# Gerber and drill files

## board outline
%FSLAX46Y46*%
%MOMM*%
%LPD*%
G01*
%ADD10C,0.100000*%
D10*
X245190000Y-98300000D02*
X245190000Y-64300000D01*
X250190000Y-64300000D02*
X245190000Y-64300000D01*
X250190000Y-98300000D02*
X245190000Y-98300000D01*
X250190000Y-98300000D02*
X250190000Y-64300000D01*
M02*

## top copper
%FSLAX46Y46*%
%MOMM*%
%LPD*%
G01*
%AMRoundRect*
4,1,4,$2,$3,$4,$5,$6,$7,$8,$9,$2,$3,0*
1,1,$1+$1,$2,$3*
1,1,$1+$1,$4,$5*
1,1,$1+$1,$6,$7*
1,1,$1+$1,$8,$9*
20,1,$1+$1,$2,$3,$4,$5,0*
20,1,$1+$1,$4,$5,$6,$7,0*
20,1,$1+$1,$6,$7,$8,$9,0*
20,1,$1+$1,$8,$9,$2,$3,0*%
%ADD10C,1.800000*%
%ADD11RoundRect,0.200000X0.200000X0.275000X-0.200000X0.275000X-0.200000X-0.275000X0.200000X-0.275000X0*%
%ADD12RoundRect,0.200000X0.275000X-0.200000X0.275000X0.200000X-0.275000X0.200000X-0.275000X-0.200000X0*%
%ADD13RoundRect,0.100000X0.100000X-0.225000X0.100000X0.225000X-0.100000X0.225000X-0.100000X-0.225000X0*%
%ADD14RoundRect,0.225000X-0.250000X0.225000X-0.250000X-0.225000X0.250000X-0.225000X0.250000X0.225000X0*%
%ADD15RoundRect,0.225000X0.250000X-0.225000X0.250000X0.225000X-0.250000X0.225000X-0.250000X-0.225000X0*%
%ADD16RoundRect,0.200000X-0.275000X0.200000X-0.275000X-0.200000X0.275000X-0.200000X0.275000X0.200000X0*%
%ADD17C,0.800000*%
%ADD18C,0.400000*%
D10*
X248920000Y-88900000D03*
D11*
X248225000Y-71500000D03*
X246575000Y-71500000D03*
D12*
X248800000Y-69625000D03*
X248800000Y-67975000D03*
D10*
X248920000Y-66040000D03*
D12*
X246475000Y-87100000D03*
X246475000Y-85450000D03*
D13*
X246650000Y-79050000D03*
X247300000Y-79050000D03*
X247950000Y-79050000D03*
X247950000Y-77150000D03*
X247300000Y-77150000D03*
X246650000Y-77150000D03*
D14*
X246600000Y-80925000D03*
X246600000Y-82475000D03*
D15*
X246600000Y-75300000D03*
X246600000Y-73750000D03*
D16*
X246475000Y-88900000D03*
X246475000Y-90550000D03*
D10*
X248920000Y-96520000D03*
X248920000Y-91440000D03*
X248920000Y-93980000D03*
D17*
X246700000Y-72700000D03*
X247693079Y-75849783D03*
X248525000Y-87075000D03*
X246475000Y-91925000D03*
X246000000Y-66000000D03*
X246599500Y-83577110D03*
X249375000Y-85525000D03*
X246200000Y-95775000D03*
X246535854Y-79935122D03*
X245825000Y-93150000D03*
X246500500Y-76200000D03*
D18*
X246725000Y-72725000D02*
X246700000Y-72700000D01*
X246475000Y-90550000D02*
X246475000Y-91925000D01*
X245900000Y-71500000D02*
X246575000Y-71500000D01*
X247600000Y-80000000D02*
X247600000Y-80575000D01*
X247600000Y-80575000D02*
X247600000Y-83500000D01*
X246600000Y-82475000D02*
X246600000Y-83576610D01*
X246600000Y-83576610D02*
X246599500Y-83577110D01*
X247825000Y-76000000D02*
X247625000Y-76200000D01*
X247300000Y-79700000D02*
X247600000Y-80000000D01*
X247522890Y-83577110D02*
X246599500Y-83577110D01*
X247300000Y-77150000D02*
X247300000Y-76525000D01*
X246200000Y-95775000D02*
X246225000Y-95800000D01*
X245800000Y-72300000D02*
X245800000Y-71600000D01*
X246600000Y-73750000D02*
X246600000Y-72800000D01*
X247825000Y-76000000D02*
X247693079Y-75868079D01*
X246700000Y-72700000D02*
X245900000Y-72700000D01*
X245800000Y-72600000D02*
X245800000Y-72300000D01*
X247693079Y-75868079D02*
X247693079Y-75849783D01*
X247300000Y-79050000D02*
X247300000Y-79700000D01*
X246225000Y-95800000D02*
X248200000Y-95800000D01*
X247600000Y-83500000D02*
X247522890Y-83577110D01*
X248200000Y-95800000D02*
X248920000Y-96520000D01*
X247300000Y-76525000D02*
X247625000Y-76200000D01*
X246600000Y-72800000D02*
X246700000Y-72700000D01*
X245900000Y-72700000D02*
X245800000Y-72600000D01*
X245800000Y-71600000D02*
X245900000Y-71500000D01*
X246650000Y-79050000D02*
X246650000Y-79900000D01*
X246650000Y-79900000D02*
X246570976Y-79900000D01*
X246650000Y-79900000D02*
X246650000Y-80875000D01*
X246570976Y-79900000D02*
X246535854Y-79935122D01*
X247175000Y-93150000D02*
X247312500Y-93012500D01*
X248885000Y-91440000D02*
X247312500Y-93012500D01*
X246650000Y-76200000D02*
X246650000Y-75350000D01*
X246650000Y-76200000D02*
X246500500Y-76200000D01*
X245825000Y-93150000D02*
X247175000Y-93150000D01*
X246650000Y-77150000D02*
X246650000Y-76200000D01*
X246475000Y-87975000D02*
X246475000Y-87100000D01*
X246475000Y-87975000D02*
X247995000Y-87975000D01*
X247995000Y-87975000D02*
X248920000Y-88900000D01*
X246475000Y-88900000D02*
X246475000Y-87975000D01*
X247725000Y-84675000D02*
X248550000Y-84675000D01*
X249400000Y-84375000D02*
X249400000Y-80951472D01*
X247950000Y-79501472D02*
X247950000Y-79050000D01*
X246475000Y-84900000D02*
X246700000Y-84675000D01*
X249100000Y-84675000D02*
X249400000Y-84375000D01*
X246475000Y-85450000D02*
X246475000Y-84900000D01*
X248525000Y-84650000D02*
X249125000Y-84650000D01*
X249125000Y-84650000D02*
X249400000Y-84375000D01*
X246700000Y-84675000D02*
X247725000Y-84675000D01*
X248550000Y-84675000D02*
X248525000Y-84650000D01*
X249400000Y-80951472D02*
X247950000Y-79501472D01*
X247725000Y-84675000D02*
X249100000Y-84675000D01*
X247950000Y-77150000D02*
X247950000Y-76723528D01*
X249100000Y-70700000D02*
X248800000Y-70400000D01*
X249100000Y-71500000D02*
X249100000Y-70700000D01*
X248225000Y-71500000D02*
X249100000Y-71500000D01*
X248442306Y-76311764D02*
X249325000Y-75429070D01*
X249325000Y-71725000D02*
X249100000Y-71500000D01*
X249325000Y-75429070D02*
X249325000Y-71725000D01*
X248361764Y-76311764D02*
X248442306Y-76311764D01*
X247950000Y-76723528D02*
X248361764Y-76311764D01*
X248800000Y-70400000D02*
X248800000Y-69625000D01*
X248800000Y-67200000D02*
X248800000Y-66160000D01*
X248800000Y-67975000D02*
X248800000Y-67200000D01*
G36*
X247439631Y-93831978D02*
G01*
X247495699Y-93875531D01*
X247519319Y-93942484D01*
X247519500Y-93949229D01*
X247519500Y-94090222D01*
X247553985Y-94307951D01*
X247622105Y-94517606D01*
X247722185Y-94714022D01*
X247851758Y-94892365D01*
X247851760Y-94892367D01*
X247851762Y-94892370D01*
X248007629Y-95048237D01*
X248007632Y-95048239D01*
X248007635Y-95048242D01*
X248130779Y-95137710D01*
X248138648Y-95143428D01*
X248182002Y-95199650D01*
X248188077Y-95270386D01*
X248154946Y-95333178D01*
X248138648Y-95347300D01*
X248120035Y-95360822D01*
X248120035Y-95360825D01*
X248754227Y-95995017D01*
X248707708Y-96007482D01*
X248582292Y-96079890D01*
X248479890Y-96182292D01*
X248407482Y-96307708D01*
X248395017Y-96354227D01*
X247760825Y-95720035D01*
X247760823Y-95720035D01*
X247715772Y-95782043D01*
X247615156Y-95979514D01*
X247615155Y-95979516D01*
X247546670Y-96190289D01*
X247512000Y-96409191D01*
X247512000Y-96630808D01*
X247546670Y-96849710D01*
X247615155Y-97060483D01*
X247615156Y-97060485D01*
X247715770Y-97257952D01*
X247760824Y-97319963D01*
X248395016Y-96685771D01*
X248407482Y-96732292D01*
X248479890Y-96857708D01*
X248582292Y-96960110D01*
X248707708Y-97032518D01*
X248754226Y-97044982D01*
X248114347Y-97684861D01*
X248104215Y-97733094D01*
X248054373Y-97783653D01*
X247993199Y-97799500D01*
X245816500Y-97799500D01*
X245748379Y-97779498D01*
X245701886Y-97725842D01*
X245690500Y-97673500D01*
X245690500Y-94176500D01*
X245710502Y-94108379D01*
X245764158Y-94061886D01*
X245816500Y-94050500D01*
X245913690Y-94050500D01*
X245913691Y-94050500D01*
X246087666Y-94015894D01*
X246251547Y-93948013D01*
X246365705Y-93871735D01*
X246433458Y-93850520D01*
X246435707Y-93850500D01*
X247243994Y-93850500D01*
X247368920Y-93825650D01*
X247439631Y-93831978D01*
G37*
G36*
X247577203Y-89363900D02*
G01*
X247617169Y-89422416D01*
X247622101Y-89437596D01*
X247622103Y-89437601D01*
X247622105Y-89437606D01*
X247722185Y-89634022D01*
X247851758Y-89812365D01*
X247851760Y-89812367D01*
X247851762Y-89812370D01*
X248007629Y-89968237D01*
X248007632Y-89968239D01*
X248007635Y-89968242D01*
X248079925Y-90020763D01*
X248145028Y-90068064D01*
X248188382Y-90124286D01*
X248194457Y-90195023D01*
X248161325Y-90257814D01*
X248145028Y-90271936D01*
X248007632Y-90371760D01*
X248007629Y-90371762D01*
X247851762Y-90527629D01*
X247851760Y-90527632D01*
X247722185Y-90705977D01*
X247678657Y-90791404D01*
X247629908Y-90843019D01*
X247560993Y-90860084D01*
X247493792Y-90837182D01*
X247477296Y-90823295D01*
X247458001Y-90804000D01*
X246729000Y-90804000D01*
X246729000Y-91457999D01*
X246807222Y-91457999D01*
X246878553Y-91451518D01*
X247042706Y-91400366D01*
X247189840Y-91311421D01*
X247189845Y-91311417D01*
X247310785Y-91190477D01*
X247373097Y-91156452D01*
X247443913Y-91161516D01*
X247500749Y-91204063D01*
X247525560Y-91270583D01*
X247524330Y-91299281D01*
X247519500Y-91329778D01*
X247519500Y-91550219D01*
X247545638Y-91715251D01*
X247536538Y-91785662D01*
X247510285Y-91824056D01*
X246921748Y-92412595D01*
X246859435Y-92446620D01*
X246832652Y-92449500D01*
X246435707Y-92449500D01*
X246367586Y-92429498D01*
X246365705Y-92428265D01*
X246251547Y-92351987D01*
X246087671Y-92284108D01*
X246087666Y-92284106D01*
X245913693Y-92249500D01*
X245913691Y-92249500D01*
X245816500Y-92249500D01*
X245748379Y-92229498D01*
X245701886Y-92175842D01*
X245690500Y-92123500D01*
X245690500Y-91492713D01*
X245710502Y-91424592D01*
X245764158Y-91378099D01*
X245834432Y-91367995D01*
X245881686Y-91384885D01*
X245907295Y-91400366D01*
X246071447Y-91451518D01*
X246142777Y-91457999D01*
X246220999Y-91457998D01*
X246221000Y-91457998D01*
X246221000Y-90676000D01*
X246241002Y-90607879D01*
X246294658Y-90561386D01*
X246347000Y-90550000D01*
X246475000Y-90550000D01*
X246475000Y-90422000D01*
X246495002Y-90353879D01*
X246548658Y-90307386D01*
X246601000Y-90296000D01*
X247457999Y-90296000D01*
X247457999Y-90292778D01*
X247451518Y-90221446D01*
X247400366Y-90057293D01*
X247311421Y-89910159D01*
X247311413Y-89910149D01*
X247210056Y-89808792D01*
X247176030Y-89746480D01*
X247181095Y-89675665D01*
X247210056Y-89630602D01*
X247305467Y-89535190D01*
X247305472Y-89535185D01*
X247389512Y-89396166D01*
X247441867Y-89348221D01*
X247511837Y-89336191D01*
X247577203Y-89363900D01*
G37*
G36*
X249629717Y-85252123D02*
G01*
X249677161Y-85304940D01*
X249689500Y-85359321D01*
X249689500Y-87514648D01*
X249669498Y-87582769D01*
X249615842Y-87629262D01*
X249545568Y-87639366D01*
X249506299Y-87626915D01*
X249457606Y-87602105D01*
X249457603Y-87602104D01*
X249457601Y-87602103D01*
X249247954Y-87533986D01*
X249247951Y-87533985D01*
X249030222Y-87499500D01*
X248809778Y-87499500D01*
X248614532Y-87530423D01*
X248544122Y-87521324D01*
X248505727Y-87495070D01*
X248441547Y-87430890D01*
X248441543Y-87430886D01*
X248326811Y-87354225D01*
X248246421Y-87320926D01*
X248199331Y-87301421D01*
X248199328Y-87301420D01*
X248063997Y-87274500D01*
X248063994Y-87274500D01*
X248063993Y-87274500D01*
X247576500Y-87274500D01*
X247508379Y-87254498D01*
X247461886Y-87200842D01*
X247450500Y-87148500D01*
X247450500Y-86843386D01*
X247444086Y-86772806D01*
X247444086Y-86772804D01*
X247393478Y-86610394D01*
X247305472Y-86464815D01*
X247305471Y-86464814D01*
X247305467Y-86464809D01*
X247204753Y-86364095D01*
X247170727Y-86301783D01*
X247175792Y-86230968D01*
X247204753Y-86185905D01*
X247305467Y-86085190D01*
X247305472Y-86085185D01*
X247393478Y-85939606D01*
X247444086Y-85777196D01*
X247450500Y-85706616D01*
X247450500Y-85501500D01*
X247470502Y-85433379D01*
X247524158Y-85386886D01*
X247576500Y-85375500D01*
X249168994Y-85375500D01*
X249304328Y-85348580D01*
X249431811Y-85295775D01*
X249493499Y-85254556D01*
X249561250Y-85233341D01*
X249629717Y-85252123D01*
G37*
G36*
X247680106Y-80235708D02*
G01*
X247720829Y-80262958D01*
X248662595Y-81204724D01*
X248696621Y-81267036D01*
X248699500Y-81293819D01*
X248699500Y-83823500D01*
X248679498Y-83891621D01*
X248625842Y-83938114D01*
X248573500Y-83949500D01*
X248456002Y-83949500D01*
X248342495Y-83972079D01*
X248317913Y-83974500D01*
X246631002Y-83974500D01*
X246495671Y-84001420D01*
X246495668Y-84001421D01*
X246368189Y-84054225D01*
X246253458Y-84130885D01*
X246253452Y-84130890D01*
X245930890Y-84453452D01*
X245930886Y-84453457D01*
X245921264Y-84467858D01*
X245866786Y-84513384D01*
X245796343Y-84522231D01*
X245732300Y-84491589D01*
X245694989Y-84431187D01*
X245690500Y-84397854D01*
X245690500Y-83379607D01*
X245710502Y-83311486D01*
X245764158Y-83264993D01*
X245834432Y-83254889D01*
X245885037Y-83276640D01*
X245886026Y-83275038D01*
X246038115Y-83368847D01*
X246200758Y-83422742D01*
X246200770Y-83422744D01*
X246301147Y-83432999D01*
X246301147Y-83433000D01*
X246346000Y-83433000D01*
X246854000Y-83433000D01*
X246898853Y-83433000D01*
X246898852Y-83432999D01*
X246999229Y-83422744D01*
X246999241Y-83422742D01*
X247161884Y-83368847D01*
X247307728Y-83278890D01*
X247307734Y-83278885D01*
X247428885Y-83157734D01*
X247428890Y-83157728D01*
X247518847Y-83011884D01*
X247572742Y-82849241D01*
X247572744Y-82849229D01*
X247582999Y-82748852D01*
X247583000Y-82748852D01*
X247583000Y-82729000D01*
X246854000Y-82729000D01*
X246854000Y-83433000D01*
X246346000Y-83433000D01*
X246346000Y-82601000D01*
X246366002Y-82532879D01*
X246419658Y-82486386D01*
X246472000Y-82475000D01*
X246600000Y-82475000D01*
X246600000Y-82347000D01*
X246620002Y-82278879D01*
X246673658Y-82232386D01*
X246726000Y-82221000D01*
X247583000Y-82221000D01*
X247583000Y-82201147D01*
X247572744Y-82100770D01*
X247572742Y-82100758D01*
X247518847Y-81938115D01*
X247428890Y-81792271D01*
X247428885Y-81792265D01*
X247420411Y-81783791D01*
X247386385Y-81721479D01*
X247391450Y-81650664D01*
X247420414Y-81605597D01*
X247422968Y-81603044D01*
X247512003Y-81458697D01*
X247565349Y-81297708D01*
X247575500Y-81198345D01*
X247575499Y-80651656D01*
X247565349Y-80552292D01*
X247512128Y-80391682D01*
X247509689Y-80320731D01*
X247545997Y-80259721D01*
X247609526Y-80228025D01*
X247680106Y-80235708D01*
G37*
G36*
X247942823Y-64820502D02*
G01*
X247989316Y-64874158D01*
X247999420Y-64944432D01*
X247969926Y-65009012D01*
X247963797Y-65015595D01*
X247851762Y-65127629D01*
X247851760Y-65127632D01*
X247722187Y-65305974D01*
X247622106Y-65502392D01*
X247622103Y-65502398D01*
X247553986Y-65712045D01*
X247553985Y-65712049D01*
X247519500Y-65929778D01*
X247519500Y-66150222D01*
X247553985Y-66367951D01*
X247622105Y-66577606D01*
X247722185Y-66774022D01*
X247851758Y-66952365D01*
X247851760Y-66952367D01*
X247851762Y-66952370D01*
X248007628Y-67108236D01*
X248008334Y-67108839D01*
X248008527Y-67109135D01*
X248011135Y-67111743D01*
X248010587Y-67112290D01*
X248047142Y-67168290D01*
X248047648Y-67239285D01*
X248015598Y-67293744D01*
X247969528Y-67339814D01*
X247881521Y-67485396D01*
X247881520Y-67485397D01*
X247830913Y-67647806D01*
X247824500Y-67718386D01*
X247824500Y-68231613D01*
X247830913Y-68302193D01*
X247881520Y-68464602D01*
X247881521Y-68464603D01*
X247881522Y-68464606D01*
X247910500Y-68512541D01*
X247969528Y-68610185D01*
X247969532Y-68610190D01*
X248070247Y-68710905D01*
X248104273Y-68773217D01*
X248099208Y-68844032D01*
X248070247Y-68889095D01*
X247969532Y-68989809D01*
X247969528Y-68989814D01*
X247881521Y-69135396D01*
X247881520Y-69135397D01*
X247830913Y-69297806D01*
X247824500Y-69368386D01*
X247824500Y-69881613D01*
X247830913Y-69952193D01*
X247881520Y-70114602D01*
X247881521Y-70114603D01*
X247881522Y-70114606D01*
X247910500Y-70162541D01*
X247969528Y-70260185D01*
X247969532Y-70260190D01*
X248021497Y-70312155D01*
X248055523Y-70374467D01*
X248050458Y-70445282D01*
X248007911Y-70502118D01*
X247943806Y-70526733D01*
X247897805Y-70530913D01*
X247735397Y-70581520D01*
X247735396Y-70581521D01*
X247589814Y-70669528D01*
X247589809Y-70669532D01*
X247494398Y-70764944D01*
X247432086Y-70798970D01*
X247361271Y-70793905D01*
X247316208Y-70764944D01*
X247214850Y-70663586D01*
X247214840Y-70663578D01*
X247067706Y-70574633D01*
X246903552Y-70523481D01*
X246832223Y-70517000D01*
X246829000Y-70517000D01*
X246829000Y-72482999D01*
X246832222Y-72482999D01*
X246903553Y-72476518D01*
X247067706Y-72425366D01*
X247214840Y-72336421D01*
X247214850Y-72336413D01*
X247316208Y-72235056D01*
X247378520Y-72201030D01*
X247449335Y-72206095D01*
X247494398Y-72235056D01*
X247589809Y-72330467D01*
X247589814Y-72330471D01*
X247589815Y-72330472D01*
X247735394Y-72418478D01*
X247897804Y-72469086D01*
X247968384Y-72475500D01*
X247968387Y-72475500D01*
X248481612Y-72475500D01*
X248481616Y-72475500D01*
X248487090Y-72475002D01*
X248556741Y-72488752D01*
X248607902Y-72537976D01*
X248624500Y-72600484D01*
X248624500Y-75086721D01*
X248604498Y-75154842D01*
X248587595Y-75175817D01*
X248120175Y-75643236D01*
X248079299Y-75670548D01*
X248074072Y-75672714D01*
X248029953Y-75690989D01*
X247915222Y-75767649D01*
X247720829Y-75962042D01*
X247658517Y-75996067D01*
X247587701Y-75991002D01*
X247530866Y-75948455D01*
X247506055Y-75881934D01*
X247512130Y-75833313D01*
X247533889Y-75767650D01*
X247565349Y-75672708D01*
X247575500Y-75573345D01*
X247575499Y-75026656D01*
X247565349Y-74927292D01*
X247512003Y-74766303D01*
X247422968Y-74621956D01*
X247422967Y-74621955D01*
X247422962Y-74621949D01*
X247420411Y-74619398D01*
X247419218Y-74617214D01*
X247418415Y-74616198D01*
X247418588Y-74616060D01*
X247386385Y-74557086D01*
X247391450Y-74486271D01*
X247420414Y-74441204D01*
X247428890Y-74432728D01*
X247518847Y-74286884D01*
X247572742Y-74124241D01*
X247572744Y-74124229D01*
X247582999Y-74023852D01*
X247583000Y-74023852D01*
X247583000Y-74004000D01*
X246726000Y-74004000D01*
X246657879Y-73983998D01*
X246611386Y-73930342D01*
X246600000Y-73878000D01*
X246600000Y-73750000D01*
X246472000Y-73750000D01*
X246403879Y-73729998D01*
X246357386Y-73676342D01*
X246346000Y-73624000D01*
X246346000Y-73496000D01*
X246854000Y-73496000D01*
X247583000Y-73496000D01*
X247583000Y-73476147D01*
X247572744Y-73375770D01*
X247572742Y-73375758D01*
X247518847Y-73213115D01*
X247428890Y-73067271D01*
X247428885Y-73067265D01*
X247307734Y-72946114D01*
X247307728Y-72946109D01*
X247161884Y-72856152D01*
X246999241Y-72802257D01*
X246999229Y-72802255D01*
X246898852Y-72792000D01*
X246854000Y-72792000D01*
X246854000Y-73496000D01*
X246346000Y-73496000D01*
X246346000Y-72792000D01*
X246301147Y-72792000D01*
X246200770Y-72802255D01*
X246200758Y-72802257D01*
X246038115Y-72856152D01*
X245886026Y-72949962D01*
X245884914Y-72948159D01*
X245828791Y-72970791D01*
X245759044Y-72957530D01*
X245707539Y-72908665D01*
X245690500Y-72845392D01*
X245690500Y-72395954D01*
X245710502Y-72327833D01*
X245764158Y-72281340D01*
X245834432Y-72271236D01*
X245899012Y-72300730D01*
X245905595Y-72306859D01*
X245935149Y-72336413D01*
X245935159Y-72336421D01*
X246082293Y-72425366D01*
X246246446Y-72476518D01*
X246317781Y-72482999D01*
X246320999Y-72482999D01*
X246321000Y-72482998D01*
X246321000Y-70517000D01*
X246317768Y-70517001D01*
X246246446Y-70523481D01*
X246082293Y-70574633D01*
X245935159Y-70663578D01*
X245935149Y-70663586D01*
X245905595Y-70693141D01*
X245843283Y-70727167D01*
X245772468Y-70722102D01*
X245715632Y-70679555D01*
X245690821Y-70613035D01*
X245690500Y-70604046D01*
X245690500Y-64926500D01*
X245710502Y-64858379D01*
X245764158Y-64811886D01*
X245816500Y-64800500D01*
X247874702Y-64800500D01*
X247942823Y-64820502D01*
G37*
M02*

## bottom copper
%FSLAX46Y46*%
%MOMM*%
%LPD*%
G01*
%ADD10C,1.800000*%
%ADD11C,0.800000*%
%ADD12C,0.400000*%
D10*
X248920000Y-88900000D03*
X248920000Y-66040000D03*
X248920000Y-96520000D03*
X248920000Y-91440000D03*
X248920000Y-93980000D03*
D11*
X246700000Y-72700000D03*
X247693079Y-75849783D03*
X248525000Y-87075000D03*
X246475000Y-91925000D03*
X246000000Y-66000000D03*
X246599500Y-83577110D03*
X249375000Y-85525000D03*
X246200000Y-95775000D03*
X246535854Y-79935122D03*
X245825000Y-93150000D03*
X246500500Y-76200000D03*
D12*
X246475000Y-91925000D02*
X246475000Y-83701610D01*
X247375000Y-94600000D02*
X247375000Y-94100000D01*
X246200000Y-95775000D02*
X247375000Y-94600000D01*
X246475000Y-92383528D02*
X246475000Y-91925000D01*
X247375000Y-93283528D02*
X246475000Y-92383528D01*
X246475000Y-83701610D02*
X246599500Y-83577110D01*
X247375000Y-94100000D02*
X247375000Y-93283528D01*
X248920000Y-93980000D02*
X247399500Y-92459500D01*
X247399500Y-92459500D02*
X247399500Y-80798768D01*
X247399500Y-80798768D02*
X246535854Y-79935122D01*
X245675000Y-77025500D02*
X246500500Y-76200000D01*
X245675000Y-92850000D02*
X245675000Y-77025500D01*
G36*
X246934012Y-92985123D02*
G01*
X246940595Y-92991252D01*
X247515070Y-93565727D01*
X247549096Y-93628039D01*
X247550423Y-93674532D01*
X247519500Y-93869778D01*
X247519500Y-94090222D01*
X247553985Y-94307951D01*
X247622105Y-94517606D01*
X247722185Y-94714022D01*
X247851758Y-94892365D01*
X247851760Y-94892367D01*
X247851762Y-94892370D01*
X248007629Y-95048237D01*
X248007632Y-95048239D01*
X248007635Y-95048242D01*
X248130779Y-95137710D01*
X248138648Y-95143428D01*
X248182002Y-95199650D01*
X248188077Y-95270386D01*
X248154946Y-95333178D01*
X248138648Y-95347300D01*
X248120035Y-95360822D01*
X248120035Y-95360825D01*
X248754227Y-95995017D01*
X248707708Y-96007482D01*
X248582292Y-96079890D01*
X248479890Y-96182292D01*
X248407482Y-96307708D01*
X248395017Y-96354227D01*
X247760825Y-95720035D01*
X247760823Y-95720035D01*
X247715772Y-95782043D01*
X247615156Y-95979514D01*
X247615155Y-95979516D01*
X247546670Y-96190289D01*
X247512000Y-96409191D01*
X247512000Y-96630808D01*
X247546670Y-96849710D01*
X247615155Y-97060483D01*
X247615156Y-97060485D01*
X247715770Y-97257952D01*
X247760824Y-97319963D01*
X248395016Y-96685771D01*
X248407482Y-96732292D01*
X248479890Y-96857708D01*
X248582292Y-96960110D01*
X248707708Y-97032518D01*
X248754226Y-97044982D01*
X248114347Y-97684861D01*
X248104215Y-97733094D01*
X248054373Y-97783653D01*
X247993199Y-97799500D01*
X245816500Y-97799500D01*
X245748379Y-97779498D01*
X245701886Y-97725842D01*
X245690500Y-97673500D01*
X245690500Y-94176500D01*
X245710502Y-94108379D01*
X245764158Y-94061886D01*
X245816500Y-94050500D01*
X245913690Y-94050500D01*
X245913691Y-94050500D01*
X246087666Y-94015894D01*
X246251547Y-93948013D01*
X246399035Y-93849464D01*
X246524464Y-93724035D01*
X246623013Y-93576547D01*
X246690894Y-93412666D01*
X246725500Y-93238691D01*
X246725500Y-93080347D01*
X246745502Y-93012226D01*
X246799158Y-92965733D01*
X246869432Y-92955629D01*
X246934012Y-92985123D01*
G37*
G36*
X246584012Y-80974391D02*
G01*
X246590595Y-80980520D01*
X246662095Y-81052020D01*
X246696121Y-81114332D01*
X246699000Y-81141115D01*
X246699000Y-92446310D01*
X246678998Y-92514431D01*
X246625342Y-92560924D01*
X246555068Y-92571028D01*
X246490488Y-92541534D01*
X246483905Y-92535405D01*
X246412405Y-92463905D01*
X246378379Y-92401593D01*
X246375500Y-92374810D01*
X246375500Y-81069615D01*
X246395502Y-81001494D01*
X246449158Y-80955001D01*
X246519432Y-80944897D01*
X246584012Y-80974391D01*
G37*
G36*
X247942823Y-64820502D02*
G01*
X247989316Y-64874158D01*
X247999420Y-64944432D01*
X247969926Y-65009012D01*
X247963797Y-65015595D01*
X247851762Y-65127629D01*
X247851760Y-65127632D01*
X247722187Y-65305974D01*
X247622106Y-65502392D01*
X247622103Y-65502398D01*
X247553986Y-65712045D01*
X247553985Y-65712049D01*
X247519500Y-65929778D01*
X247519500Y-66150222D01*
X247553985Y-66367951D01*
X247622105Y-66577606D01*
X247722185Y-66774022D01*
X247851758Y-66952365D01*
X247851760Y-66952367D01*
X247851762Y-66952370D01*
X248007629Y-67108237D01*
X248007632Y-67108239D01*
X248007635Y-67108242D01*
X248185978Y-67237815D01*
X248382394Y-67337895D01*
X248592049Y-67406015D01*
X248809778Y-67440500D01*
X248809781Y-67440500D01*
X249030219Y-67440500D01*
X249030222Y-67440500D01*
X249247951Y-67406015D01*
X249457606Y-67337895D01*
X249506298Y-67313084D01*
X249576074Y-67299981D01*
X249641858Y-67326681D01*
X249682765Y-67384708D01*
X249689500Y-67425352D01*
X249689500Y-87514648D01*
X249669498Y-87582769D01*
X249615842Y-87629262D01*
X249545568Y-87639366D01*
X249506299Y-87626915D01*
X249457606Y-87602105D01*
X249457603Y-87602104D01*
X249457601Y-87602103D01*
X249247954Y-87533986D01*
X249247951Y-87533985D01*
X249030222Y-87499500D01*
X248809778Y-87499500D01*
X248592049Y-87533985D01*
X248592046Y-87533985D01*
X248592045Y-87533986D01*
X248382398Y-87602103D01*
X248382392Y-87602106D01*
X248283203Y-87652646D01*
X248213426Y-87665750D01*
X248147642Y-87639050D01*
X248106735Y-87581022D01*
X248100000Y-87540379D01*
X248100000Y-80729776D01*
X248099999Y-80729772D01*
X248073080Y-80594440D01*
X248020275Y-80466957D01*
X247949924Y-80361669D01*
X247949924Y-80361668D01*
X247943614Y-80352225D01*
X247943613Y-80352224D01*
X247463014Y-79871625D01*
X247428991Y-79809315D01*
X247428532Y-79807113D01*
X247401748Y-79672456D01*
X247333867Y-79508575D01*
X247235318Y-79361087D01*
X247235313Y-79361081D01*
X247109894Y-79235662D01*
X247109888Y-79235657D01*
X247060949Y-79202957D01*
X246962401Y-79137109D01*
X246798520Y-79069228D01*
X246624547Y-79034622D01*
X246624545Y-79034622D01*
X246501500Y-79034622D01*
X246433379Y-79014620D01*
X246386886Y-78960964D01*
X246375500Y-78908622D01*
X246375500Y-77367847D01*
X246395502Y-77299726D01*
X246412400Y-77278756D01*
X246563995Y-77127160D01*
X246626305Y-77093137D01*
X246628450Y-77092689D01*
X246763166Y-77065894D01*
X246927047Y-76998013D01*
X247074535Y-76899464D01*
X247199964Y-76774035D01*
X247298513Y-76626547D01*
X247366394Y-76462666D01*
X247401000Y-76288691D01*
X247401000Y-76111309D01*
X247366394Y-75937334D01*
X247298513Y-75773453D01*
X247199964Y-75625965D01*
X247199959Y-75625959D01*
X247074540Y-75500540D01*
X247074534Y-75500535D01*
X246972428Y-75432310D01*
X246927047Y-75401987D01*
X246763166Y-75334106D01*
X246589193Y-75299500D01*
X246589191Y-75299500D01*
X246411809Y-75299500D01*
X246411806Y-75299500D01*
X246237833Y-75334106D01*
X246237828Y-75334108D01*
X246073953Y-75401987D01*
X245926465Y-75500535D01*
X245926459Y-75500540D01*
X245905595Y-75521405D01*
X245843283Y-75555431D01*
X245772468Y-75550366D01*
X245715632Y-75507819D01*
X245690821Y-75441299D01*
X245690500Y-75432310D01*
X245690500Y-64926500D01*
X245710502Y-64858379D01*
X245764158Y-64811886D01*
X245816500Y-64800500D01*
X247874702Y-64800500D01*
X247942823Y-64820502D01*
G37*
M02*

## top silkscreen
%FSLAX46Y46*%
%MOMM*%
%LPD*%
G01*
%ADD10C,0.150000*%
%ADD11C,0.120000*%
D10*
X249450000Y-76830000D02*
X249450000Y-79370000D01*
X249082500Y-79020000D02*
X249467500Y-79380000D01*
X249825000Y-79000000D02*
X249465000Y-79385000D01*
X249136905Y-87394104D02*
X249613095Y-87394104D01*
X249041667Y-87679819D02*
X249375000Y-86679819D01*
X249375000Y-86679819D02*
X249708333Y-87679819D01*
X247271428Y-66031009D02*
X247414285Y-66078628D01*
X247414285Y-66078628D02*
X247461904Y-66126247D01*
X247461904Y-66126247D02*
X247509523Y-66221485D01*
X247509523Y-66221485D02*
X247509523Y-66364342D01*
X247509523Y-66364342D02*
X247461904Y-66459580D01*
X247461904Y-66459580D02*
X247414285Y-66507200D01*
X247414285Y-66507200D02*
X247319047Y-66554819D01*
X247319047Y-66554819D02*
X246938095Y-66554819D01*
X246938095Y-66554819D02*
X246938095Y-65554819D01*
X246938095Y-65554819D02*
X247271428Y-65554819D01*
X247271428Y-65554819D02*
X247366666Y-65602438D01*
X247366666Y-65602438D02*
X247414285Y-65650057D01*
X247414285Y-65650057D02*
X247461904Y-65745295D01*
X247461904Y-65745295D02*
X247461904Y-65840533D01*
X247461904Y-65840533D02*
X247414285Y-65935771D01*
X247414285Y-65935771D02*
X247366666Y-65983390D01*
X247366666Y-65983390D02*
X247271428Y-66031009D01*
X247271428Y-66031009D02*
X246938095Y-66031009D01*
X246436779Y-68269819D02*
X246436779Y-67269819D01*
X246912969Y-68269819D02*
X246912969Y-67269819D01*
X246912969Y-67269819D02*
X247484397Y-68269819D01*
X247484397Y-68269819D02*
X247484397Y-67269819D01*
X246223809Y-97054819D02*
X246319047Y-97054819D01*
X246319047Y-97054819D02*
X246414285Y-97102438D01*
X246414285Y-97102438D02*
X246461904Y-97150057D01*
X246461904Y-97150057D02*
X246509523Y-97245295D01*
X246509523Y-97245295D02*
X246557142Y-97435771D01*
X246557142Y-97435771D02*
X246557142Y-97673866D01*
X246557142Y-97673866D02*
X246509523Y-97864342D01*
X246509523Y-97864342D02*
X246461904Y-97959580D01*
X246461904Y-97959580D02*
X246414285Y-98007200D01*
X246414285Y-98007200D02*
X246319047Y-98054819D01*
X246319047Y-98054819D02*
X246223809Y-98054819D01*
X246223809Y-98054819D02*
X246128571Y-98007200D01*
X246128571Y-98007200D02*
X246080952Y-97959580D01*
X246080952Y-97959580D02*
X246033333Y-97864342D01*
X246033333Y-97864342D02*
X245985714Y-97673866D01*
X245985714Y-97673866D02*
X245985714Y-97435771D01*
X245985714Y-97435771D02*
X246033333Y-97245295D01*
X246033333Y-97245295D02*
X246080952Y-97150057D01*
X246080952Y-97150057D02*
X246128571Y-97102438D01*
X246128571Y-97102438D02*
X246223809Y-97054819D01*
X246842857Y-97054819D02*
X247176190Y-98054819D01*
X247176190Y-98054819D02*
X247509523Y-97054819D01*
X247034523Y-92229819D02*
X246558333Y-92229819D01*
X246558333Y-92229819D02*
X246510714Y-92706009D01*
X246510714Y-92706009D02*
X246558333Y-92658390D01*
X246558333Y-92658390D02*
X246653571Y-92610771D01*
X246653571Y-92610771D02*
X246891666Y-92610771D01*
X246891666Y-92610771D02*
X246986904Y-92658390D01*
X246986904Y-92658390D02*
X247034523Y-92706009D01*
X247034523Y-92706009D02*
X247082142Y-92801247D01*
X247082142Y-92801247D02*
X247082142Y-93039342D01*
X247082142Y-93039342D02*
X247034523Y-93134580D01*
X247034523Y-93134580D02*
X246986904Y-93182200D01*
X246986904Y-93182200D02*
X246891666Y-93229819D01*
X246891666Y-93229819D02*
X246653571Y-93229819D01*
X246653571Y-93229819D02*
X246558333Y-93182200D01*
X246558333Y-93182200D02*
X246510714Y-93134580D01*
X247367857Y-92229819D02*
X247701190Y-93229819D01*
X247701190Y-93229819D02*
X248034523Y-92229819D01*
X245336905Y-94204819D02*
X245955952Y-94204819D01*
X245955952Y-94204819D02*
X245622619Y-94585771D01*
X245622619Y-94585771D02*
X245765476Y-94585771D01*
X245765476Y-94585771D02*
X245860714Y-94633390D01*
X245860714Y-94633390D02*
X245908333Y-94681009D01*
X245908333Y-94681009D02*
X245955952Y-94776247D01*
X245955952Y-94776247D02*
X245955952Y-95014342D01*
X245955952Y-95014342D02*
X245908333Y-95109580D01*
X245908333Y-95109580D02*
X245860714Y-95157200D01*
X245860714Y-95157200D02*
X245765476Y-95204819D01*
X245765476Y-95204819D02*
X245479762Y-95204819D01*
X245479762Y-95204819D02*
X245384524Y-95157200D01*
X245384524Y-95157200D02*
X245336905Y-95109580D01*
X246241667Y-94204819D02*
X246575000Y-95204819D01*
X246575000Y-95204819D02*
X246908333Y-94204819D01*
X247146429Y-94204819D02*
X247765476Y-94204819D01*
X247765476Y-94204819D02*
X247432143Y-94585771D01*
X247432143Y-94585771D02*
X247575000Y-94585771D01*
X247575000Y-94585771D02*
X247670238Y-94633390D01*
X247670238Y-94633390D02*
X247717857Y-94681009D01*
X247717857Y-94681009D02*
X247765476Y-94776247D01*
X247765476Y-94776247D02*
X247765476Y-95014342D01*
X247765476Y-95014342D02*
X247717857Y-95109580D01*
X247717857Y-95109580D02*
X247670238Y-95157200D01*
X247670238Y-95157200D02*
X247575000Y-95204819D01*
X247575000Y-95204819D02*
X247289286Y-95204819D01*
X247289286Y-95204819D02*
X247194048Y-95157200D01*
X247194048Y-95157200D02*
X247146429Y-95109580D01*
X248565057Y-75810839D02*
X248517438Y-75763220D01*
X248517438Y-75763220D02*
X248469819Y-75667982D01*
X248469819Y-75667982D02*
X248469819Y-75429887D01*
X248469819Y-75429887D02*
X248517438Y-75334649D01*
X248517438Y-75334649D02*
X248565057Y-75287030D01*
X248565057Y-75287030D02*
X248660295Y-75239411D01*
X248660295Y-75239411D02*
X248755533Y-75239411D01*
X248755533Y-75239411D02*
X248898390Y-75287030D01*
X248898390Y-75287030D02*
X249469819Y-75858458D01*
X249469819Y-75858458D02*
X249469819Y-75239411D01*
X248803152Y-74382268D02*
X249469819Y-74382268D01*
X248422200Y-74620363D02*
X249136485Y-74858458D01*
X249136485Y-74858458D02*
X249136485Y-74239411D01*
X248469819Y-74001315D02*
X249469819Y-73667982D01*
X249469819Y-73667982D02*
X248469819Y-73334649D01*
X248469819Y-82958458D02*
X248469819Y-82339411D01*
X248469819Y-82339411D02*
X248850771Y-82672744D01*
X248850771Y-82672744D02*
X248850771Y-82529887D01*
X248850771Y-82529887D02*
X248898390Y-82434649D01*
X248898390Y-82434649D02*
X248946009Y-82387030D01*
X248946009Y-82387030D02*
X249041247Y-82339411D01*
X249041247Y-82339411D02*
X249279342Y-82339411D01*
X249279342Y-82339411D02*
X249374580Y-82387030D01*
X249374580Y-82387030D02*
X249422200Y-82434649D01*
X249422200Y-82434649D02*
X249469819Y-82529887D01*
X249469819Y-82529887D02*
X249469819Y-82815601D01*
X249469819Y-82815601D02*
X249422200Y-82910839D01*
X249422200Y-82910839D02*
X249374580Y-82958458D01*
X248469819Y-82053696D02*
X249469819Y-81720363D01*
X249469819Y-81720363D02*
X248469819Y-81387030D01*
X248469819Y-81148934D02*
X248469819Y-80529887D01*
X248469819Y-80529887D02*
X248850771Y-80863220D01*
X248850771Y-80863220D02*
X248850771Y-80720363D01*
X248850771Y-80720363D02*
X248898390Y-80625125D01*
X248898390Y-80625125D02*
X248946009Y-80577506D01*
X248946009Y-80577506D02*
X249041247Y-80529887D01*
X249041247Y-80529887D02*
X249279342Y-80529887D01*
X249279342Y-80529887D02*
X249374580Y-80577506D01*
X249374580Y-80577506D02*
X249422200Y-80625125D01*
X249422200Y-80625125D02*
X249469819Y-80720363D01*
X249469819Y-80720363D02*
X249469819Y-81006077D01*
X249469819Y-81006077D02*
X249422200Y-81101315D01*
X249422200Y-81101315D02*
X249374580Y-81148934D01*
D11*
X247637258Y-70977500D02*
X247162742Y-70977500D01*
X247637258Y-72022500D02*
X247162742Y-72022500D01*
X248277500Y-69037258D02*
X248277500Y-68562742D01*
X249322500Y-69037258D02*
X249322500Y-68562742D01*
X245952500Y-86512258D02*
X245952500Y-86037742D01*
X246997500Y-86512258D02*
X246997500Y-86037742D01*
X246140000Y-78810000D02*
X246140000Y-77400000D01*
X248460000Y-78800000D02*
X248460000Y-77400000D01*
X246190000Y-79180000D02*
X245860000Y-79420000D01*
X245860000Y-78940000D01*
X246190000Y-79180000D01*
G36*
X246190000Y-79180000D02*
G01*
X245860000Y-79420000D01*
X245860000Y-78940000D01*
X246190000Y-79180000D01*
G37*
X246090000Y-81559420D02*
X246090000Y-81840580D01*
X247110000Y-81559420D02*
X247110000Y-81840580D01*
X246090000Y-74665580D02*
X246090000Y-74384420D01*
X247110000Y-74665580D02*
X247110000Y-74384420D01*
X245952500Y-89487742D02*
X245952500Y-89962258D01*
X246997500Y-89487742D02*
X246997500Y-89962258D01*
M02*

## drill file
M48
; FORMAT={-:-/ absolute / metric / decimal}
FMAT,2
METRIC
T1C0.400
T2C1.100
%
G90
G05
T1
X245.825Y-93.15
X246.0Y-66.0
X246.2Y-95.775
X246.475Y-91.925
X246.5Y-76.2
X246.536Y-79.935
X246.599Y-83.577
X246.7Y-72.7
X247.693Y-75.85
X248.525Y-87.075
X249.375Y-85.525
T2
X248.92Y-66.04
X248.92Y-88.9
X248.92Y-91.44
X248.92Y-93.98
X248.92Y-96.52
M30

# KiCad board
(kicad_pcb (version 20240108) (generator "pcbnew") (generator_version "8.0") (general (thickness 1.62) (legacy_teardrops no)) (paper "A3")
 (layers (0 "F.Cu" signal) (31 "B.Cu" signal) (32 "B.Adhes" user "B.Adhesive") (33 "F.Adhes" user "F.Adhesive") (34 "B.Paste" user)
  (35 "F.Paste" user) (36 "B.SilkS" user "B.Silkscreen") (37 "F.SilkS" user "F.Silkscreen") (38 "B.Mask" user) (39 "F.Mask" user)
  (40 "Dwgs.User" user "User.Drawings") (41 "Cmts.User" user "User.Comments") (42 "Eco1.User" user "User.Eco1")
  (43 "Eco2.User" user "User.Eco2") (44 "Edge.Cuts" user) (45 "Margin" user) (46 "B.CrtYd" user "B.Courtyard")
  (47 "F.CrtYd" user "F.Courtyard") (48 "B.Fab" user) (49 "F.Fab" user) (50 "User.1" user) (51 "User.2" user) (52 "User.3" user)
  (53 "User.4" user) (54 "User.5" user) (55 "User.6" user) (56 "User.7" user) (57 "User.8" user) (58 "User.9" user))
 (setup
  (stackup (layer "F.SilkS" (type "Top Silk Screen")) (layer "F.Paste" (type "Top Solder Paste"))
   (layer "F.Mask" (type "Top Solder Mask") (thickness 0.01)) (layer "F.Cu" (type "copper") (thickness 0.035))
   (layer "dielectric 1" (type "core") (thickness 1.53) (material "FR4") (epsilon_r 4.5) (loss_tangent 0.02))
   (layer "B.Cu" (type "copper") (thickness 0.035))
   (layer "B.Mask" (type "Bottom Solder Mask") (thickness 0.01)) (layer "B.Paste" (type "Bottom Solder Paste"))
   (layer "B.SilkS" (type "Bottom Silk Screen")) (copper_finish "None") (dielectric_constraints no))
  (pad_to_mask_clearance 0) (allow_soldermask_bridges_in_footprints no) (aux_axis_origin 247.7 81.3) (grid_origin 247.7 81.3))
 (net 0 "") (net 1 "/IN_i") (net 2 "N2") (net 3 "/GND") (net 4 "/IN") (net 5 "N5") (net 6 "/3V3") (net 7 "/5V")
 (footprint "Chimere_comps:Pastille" (layer "F.Cu") (at 248.92 88.9)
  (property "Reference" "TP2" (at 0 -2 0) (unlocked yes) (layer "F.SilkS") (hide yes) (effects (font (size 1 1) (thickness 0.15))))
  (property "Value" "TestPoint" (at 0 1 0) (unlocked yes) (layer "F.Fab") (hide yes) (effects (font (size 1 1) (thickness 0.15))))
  (pad "1" thru_hole circle (at 0 0) (size 1.8 1.8) (drill 1.1) (layers "*.Cu" "*.Mask") (remove_unused_layers no) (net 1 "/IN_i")))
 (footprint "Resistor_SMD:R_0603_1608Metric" (layer "F.Cu") (at 247.4 71.5 180)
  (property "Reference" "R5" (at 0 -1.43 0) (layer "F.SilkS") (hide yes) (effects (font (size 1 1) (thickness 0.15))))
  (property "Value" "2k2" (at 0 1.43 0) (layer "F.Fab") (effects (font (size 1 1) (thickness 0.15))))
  (fp_line (start -0.237258 0.5225) (end 0.237258 0.5225) (stroke (width 0.12) (type solid)) (layer "F.SilkS"))
  (fp_line (start -0.237258 -0.5225) (end 0.237258 -0.5225) (stroke (width 0.12) (type solid)) (layer "F.SilkS"))
  (pad "1" smd roundrect (at -0.825 0 180) (size 0.8 0.95) (layers "F.Cu" "F.Paste" "F.Mask") (roundrect_rratio 0.25) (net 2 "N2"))
  (pad "2" smd roundrect (at 0.825 0 180) (size 0.8 0.95) (layers "F.Cu" "F.Paste" "F.Mask") (roundrect_rratio 0.25) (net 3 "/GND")))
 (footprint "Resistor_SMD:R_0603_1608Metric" (layer "F.Cu") (at 248.8 68.8 90)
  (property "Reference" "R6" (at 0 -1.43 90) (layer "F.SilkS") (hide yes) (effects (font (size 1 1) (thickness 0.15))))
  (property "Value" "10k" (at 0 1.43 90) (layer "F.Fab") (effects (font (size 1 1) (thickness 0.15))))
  (fp_line (start -0.237258 -0.5225) (end 0.237258 -0.5225) (stroke (width 0.12) (type solid)) (layer "F.SilkS"))
  (fp_line (start -0.237258 0.5225) (end 0.237258 0.5225) (stroke (width 0.12) (type solid)) (layer "F.SilkS"))
  (pad "1" smd roundrect (at -0.825 0 90) (size 0.8 0.95) (layers "F.Cu" "F.Paste" "F.Mask") (roundrect_rratio 0.25) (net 2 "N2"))
  (pad "2" smd roundrect (at 0.825 0 90) (size 0.8 0.95) (layers "F.Cu" "F.Paste" "F.Mask") (roundrect_rratio 0.25) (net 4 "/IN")))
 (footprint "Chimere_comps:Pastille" (layer "F.Cu") (at 248.92 66.04)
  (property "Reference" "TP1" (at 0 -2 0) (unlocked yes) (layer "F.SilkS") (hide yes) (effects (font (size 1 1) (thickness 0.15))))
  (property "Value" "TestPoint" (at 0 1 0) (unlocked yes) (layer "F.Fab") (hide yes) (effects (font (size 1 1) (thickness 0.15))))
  (pad "1" thru_hole circle (at 0 0) (size 1.8 1.8) (drill 1.1) (layers "*.Cu" "*.Mask") (remove_unused_layers no) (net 4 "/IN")))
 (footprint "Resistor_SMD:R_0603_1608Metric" (layer "F.Cu") (at 246.475 86.275 90)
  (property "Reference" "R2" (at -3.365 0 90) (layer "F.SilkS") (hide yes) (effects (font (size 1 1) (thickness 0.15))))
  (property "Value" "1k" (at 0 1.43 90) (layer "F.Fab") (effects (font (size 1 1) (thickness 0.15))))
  (fp_line (start -0.237258 -0.5225) (end 0.237258 -0.5225) (stroke (width 0.12) (type solid)) (layer "F.SilkS"))
  (fp_line (start -0.237258 0.5225) (end 0.237258 0.5225) (stroke (width 0.12) (type solid)) (layer "F.SilkS"))
  (pad "1" smd roundrect (at -0.825 0 90) (size 0.8 0.95) (layers "F.Cu" "F.Paste" "F.Mask") (roundrect_rratio 0.25) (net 1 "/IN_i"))
  (pad "2" smd roundrect (at 0.825 0 90) (size 0.8 0.95) (layers "F.Cu" "F.Paste" "F.Mask") (roundrect_rratio 0.25) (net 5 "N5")))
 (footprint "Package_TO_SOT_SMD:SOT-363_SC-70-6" (layer "F.Cu") (at 247.3 78.1 90)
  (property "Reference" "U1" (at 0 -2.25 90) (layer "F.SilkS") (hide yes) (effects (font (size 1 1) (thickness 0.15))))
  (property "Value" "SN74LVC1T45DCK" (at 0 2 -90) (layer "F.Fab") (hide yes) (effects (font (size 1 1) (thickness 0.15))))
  (fp_line (start -0.71 -1.16) (end 0.7 -1.16) (stroke (width 0.12) (type solid)) (layer "F.SilkS"))
  (fp_line (start -0.7 1.16) (end 0.7 1.16) (stroke (width 0.12) (type solid)) (layer "F.SilkS"))
  (fp_poly
   (pts (xy -1.08 -1.11) (xy -1.32 -1.44) (xy -0.84 -1.44) (xy -1.08 -1.11)) (stroke (width 0.12) (type solid)) (fill solid)
   (layer "F.SilkS"))
  (pad "1" smd roundrect (at -0.95 -0.65 90) (size 0.65 0.4) (layers "F.Cu" "F.Paste" "F.Mask") (roundrect_rratio 0.25) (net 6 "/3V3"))
  (pad "2" smd roundrect (at -0.95 0 90) (size 0.65 0.4) (layers "F.Cu" "F.Paste" "F.Mask") (roundrect_rratio 0.25) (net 3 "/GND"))
  (pad "3" smd roundrect (at -0.95 0.65 90) (size 0.65 0.4) (layers "F.Cu" "F.Paste" "F.Mask") (roundrect_rratio 0.25) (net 5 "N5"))
  (pad "4" smd roundrect (at 0.95 0.65 90) (size 0.65 0.4) (layers "F.Cu" "F.Paste" "F.Mask") (roundrect_rratio 0.25) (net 2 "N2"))
  (pad "5" smd roundrect (at 0.95 0 90) (size 0.65 0.4) (layers "F.Cu" "F.Paste" "F.Mask") (roundrect_rratio 0.25) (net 3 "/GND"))
  (pad "6" smd roundrect (at 0.95 -0.65 90) (size 0.65 0.4) (layers "F.Cu" "F.Paste" "F.Mask") (roundrect_rratio 0.25) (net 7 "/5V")))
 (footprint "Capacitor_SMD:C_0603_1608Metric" (layer "F.Cu") (at 246.6 81.7 -90)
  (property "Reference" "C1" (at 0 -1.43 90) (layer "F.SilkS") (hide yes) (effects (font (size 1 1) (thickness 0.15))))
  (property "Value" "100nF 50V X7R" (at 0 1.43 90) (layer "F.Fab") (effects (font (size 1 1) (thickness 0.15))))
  (fp_line (start -0.14058 0.51) (end 0.14058 0.51) (stroke (width 0.12) (type solid)) (layer "F.SilkS"))
  (fp_line (start -0.14058 -0.51) (end 0.14058 -0.51) (stroke (width 0.12) (type solid)) (layer "F.SilkS"))
  (pad "1" smd roundrect (at -0.775 0 270) (size 0.9 0.95) (layers "F.Cu" "F.Paste" "F.Mask") (roundrect_rratio 0.25) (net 6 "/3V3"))
  (pad "2" smd roundrect (at 0.775 0 270) (size 0.9 0.95) (layers "F.Cu" "F.Paste" "F.Mask") (roundrect_rratio 0.25) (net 3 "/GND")))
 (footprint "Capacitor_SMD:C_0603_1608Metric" (layer "F.Cu") (at 246.6 74.525 90)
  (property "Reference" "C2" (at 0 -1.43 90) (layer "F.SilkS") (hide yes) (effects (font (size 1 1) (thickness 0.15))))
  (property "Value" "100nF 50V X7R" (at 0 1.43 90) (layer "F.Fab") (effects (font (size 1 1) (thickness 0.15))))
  (fp_line (start -0.14058 -0.51) (end 0.14058 -0.51) (stroke (width 0.12) (type solid)) (layer "F.SilkS"))
  (fp_line (start -0.14058 0.51) (end 0.14058 0.51) (stroke (width 0.12) (type solid)) (layer "F.SilkS"))
  (pad "1" smd roundrect (at -0.775 0 90) (size 0.9 0.95) (layers "F.Cu" "F.Paste" "F.Mask") (roundrect_rratio 0.25) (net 7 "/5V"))
  (pad "2" smd roundrect (at 0.775 0 90) (size 0.9 0.95) (layers "F.Cu" "F.Paste" "F.Mask") (roundrect_rratio 0.25) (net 3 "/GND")))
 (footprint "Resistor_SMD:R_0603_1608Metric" (layer "F.Cu") (at 246.475 89.725 -90)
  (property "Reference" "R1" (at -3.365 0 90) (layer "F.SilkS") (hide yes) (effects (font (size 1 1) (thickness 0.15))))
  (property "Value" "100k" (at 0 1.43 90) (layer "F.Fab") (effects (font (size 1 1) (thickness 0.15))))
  (fp_line (start -0.237258 0.5225) (end 0.237258 0.5225) (stroke (width 0.12) (type solid)) (layer "F.SilkS"))
  (fp_line (start -0.237258 -0.5225) (end 0.237258 -0.5225) (stroke (width 0.12) (type solid)) (layer "F.SilkS"))
  (pad "1" smd roundrect (at -0.825 0 270) (size 0.8 0.95) (layers "F.Cu" "F.Paste" "F.Mask") (roundrect_rratio 0.25) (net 1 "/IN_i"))
  (pad "2" smd roundrect (at 0.825 0 270) (size 0.8 0.95) (layers "F.Cu" "F.Paste" "F.Mask") (roundrect_rratio 0.25) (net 3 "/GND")))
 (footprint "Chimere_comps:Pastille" (layer "F.Cu") (at 248.92 96.52)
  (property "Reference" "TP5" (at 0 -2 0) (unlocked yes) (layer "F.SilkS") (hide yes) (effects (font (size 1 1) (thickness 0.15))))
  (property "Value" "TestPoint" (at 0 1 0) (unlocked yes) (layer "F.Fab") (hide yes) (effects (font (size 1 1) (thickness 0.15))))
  (pad "1" thru_hole circle (at 0 0) (size 1.8 1.8) (drill 1.1) (layers "*.Cu" "*.Mask") (remove_unused_layers no) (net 3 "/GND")))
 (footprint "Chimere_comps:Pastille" (layer "F.Cu") (at 248.92 91.44)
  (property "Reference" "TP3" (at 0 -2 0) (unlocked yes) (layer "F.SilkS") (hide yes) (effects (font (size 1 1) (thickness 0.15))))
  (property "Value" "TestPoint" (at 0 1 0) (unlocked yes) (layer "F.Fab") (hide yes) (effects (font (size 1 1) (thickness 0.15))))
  (pad "1" thru_hole circle (at 0 0) (size 1.8 1.8) (drill 1.1) (layers "*.Cu" "*.Mask") (remove_unused_layers no) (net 7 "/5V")))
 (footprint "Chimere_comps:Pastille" (layer "F.Cu") (at 248.92 93.98)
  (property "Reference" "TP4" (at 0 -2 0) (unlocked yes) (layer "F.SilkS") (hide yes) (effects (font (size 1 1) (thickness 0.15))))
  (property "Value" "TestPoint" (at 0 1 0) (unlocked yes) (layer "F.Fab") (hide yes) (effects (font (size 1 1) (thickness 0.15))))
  (pad "1" thru_hole circle (at 0 0) (size 1.8 1.8) (drill 1.1) (layers "*.Cu" "*.Mask") (remove_unused_layers no) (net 6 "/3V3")))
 (gr_line (start 249.45 76.83) (end 249.45 79.37) (stroke (width 0.15) (type solid)) (layer "F.SilkS"))
 (gr_line (start 249.0825 79.02) (end 249.4675 79.38) (stroke (width 0.15) (type solid)) (layer "F.SilkS"))
 (gr_line (start 249.825 79) (end 249.465 79.385) (stroke (width 0.15) (type solid)) (layer "F.SilkS"))
 (gr_line (start 245.19 98.3) (end 245.19 64.3) (stroke (width 0.1) (type default)) (layer "Edge.Cuts"))
 (gr_line (start 250.19 64.3) (end 245.19 64.3) (stroke (width 0.1) (type default)) (layer "Edge.Cuts"))
 (gr_line (start 250.19 98.3) (end 245.19 98.3) (stroke (width 0.1) (type default)) (layer "Edge.Cuts"))
 (gr_line (start 250.19 98.3) (end 250.19 64.3) (stroke (width 0.1) (type default)) (layer "Edge.Cuts"))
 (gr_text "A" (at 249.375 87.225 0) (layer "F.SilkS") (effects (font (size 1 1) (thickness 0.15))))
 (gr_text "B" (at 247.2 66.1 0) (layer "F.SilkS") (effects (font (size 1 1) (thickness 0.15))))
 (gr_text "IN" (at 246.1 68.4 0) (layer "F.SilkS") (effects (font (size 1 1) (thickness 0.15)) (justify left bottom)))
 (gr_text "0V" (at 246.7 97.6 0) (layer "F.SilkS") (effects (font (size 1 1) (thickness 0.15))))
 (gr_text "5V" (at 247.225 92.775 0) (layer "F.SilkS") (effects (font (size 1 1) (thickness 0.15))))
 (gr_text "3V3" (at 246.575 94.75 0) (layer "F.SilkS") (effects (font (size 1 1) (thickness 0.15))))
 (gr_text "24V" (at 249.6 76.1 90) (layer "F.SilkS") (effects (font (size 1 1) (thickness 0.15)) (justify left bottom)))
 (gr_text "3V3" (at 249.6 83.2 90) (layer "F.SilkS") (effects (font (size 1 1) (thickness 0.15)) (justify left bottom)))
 (segment (start 246.725 72.725) (end 246.7 72.7) (width 0.4) (layer "F.Cu") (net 3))
 (segment (start 246.475 90.55) (end 246.475 91.925) (width 0.4) (layer "F.Cu") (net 3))
 (segment (start 245.9 71.5) (end 246.575 71.5) (width 0.4) (layer "F.Cu") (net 3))
 (segment (start 247.6 80) (end 247.6 80.575) (width 0.4) (layer "F.Cu") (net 3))
 (segment (start 247.6 80.575) (end 247.6 83.5) (width 0.4) (layer "F.Cu") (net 3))
 (segment (start 246.6 82.475) (end 246.6 83.57661) (width 0.4) (layer "F.Cu") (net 3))
 (segment (start 246.6 83.57661) (end 246.5995 83.57711) (width 0.4) (layer "F.Cu") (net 3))
 (segment (start 247.825 76) (end 247.625 76.2) (width 0.4) (layer "F.Cu") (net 3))
 (segment (start 247.3 79.7) (end 247.6 80) (width 0.4) (layer "F.Cu") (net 3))
 (segment (start 247.52289 83.57711) (end 246.5995 83.57711) (width 0.4) (layer "F.Cu") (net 3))
 (segment (start 247.3 77.15) (end 247.3 76.525) (width 0.4) (layer "F.Cu") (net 3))
 (segment (start 246.2 95.775) (end 246.225 95.8) (width 0.4) (layer "F.Cu") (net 3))
 (segment (start 245.8 72.3) (end 245.8 71.6) (width 0.4) (layer "F.Cu") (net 3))
 (segment (start 246.6 73.75) (end 246.6 72.8) (width 0.4) (layer "F.Cu") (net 3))
 (segment (start 247.825 76) (end 247.693079 75.868079) (width 0.4) (layer "F.Cu") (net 3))
 (segment (start 246.7 72.7) (end 245.9 72.7) (width 0.4) (layer "F.Cu") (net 3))
 (segment (start 245.8 72.6) (end 245.8 72.3) (width 0.4) (layer "F.Cu") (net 3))
 (segment (start 247.693079 75.868079) (end 247.693079 75.849783) (width 0.4) (layer "F.Cu") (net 3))
 (segment (start 247.3 79.05) (end 247.3 79.7) (width 0.4) (layer "F.Cu") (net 3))
 (segment (start 246.225 95.8) (end 248.2 95.8) (width 0.4) (layer "F.Cu") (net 3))
 (segment (start 247.6 83.5) (end 247.52289 83.57711) (width 0.4) (layer "F.Cu") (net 3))
 (segment (start 248.2 95.8) (end 248.92 96.52) (width 0.4) (layer "F.Cu") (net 3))
 (segment (start 247.3 76.525) (end 247.625 76.2) (width 0.4) (layer "F.Cu") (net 3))
 (segment (start 246.6 72.8) (end 246.7 72.7) (width 0.4) (layer "F.Cu") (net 3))
 (segment (start 245.9 72.7) (end 245.8 72.6) (width 0.4) (layer "F.Cu") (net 3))
 (segment (start 245.8 71.6) (end 245.9 71.5) (width 0.4) (layer "F.Cu") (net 3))
 (via (at 246.7 72.7) (size 0.8) (drill 0.4) (layers "F.Cu" "B.Cu") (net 3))
 (via (at 247.693079 75.849783) (size 0.8) (drill 0.4) (layers "F.Cu" "B.Cu") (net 3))
 (via (at 248.525 87.075) (size 0.8) (drill 0.4) (layers "F.Cu" "B.Cu") (free yes) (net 3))
 (via (at 246.475 91.925) (size 0.8) (drill 0.4) (layers "F.Cu" "B.Cu") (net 3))
 (via (at 246 66) (size 0.8) (drill 0.4) (layers "F.Cu" "B.Cu") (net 3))
 (via (at 246.5995 83.57711) (size 0.8) (drill 0.4) (layers "F.Cu" "B.Cu") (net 3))
 (via (at 249.375 85.525) (size 0.8) (drill 0.4) (layers "F.Cu" "B.Cu") (free yes) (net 3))
 (via (at 246.2 95.775) (size 0.8) (drill 0.4) (layers "F.Cu" "B.Cu") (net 3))
 (segment (start 246.475 91.925) (end 246.475 83.70161) (width 0.4) (layer "B.Cu") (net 3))
 (segment (start 247.375 94.6) (end 247.375 94.1) (width 0.4) (layer "B.Cu") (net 3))
 (segment (start 246.2 95.775) (end 247.375 94.6) (width 0.4) (layer "B.Cu") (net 3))
 (segment (start 246.475 92.383528) (end 246.475 91.925) (width 0.4) (layer "B.Cu") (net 3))
 (segment (start 247.375 93.283528) (end 246.475 92.383528) (width 0.4) (layer "B.Cu") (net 3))
 (segment (start 246.475 83.70161) (end 246.5995 83.57711) (width 0.4) (layer "B.Cu") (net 3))
 (segment (start 247.375 94.1) (end 247.375 93.283528) (width 0.4) (layer "B.Cu") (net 3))
 (segment (start 246.65 79.05) (end 246.65 79.9) (width 0.4) (layer "F.Cu") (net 6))
 (segment (start 246.65 79.9) (end 246.570976 79.9) (width 0.4) (layer "F.Cu") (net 6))
 (segment (start 246.65 79.9) (end 246.65 80.875) (width 0.4) (layer "F.Cu") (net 6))
 (segment (start 246.570976 79.9) (end 246.535854 79.935122) (width 0.4) (layer "F.Cu") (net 6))
 (via (at 246.535854 79.935122) (size 0.8) (drill 0.4) (layers "F.Cu" "B.Cu") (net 6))
 (segment (start 248.92 93.98) (end 247.3995 92.4595) (width 0.4) (layer "B.Cu") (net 6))
 (segment (start 247.3995 92.4595) (end 247.3995 80.798768) (width 0.4) (layer "B.Cu") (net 6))
 (segment (start 247.3995 80.798768) (end 246.535854 79.935122) (width 0.4) (layer "B.Cu") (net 6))
 (segment (start 247.175 93.15) (end 247.3125 93.0125) (width 0.4) (layer "F.Cu") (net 7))
 (segment (start 248.885 91.44) (end 247.3125 93.0125) (width 0.4) (layer "F.Cu") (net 7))
 (segment (start 246.65 76.2) (end 246.65 75.35) (width 0.4) (layer "F.Cu") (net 7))
 (segment (start 246.65 76.2) (end 246.5005 76.2) (width 0.4) (layer "F.Cu") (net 7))
 (segment (start 245.825 93.15) (end 247.175 93.15) (width 0.4) (layer "F.Cu") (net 7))
 (segment (start 246.65 77.15) (end 246.65 76.2) (width 0.4) (layer "F.Cu") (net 7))
 (via (at 245.825 93.15) (size 0.8) (drill 0.4) (layers "F.Cu" "B.Cu") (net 7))
 (via (at 246.5005 76.2) (size 0.8) (drill 0.4) (layers "F.Cu" "B.Cu") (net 7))
 (segment (start 245.675 77.0255) (end 246.5005 76.2) (width 0.4) (layer "B.Cu") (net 7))
 (segment (start 245.675 92.85) (end 245.675 77.0255) (width 0.4) (layer "B.Cu") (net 7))
 (segment (start 246.475 87.975) (end 246.475 87.1) (width 0.4) (layer "F.Cu") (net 1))
 (segment (start 246.475 87.975) (end 247.995 87.975) (width 0.4) (layer "F.Cu") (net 1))
 (segment (start 247.995 87.975) (end 248.92 88.9) (width 0.4) (layer "F.Cu") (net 1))
 (segment (start 246.475 88.9) (end 246.475 87.975) (width 0.4) (layer "F.Cu") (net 1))
 (segment (start 247.725 84.675) (end 248.55 84.675) (width 0.4) (layer "F.Cu") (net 5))
 (segment (start 249.4 84.375) (end 249.4 80.951472) (width 0.4) (layer "F.Cu") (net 5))
 (segment (start 247.95 79.501472) (end 247.95 79.05) (width 0.4) (layer "F.Cu") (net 5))
 (segment (start 246.475 84.9) (end 246.7 84.675) (width 0.4) (layer "F.Cu") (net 5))
 (segment (start 249.1 84.675) (end 249.4 84.375) (width 0.4) (layer "F.Cu") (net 5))
 (segment (start 246.475 85.45) (end 246.475 84.9) (width 0.4) (layer "F.Cu") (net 5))
 (segment (start 248.525 84.65) (end 249.125 84.65) (width 0.4) (layer "F.Cu") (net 5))
 (segment (start 249.125 84.65) (end 249.4 84.375) (width 0.4) (layer "F.Cu") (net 5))
 (segment (start 246.7 84.675) (end 247.725 84.675) (width 0.4) (layer "F.Cu") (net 5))
 (segment (start 248.55 84.675) (end 248.525 84.65) (width 0.4) (layer "F.Cu") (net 5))
 (segment (start 249.4 80.951472) (end 247.95 79.501472) (width 0.4) (layer "F.Cu") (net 5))
 (segment (start 247.725 84.675) (end 249.1 84.675) (width 0.4) (layer "F.Cu") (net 5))
 (segment (start 247.95 77.15) (end 247.95 76.723528) (width 0.4) (layer "F.Cu") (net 2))
 (segment (start 249.1 70.7) (end 248.8 70.4) (width 0.4) (layer "F.Cu") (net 2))
 (segment (start 249.1 71.5) (end 249.1 70.7) (width 0.4) (layer "F.Cu") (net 2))
 (segment (start 248.225 71.5) (end 249.1 71.5) (width 0.4) (layer "F.Cu") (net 2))
 (segment (start 248.442306 76.311764) (end 249.325 75.42907) (width 0.4) (layer "F.Cu") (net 2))
 (segment (start 249.325 71.725) (end 249.1 71.5) (width 0.4) (layer "F.Cu") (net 2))
 (segment (start 249.325 75.42907) (end 249.325 71.725) (width 0.4) (layer "F.Cu") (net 2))
 (segment (start 248.361764 76.311764) (end 248.442306 76.311764) (width 0.4) (layer "F.Cu") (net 2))
 (segment (start 247.95 76.723528) (end 248.361764 76.311764) (width 0.4) (layer "F.Cu") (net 2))
 (segment (start 248.8 70.4) (end 248.8 69.625) (width 0.4) (layer "F.Cu") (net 2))
 (segment (start 248.8 67.2) (end 248.8 66.16) (width 0.4) (layer "F.Cu") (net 4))
 (segment (start 248.8 67.975) (end 248.8 67.2) (width 0.4) (layer "F.Cu") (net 4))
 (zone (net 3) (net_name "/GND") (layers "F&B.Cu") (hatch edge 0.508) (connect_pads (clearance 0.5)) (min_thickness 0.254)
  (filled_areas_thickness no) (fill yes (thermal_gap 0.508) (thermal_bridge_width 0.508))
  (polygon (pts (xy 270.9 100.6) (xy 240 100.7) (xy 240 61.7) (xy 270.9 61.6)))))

